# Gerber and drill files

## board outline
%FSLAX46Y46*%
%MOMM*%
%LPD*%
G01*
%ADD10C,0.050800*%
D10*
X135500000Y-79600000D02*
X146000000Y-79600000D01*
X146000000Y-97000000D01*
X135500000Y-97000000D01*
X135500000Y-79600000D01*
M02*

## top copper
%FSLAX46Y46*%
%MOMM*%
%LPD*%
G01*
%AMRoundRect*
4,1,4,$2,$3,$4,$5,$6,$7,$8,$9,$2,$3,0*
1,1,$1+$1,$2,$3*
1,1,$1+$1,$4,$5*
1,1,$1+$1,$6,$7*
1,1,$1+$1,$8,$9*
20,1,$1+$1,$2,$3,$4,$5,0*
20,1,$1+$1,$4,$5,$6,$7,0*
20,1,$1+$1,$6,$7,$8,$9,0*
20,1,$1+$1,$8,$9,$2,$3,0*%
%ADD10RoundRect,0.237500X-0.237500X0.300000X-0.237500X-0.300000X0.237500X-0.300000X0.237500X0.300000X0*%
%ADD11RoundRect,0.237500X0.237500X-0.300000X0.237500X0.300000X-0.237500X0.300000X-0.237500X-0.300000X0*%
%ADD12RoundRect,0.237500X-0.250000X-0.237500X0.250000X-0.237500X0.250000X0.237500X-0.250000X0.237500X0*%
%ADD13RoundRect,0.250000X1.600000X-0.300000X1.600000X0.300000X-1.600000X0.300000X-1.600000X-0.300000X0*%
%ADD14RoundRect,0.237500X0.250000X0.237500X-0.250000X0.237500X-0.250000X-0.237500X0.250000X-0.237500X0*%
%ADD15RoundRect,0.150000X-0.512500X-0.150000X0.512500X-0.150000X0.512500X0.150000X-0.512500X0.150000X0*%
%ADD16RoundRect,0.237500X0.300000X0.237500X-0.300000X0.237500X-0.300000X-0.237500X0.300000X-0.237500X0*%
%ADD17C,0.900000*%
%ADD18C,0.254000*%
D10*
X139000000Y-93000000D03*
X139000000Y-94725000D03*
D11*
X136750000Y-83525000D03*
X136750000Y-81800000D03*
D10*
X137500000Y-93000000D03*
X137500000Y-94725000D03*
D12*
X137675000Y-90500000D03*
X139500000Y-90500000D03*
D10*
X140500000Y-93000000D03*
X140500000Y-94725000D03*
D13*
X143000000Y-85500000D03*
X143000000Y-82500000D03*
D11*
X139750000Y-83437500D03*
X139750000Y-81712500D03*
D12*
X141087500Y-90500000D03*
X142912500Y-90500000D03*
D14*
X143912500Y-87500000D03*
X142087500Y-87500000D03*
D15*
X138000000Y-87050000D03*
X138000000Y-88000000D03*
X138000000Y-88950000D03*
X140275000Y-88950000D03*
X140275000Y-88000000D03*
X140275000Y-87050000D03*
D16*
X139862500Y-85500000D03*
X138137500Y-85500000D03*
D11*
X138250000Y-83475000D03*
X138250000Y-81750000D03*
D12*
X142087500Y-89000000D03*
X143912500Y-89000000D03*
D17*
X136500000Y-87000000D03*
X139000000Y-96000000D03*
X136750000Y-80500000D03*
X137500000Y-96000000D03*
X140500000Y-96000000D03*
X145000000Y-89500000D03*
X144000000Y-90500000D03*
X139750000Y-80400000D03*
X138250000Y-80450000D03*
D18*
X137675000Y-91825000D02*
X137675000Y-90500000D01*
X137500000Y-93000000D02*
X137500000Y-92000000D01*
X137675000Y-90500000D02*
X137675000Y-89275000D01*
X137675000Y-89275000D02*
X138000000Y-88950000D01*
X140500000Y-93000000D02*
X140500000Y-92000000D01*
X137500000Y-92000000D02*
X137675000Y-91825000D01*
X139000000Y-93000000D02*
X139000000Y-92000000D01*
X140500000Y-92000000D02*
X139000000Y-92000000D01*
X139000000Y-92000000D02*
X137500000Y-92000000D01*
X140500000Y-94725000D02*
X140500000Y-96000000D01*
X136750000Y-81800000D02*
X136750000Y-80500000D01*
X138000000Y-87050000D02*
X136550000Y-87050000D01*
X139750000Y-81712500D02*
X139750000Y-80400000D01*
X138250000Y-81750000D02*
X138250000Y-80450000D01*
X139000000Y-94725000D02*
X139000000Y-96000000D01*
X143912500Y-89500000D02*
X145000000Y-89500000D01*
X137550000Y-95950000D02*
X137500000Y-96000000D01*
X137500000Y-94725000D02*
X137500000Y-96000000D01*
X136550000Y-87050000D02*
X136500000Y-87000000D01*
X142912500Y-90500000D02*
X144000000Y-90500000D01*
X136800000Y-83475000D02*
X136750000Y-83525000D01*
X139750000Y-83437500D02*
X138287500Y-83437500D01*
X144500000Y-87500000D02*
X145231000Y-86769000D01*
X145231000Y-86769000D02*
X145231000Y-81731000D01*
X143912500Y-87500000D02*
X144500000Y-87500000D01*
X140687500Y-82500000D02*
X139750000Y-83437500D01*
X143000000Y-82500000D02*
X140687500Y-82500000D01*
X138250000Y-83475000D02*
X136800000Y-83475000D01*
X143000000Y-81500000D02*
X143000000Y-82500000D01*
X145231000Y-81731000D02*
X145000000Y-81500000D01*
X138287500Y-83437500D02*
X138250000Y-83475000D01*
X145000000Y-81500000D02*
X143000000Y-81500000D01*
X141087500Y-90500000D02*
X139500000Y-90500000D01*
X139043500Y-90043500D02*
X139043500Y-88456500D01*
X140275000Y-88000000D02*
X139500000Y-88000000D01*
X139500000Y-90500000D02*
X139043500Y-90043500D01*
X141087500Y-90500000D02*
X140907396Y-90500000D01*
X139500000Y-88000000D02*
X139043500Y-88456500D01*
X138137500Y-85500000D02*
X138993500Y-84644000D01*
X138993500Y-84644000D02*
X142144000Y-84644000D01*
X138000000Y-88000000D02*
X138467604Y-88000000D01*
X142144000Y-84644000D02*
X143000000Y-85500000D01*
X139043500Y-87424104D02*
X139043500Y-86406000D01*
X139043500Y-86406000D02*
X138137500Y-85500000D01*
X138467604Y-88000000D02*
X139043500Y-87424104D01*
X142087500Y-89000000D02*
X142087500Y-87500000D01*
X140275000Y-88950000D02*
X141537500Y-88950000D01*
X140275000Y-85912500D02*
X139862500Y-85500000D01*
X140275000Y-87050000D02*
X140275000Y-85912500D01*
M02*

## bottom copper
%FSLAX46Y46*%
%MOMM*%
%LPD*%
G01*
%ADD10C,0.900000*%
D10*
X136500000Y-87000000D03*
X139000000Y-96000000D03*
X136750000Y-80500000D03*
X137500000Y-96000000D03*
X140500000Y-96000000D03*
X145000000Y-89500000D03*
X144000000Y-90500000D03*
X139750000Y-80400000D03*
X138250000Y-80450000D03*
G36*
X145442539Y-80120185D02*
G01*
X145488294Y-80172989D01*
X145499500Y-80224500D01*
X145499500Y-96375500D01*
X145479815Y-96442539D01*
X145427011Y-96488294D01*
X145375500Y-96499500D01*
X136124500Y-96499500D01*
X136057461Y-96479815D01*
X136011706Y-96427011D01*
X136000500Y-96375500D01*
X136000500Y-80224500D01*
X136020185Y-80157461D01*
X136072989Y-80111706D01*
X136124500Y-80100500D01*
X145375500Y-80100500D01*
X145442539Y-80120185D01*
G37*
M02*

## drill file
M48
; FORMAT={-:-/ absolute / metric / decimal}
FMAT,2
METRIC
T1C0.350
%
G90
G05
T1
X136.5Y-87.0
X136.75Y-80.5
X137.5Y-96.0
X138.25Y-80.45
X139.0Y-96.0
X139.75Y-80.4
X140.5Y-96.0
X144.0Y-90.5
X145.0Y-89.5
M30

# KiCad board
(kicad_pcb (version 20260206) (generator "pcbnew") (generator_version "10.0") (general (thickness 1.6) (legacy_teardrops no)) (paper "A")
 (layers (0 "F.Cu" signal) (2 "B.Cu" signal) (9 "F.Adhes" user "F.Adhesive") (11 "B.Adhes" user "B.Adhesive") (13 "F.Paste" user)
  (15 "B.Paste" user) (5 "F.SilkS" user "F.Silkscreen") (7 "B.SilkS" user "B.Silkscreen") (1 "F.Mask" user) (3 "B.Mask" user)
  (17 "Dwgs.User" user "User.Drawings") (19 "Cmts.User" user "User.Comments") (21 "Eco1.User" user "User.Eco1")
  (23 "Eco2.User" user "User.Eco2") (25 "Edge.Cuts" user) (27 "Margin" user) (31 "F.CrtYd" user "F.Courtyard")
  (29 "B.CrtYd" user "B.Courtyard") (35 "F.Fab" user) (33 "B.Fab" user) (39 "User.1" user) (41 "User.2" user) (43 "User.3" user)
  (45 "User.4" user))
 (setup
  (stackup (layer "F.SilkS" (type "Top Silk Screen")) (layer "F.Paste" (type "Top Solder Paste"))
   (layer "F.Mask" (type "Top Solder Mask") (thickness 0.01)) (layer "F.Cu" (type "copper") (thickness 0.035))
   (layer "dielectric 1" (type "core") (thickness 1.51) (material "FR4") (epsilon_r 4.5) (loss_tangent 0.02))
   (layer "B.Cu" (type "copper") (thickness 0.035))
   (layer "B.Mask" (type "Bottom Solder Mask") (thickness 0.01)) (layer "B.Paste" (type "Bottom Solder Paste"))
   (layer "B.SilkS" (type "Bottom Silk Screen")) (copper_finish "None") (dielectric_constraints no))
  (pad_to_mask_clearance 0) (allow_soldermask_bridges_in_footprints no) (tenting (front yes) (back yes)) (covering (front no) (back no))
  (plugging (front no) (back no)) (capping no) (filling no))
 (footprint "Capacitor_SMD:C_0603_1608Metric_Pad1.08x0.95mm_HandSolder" (layer "F.Cu") (at 139 93.8625 -90)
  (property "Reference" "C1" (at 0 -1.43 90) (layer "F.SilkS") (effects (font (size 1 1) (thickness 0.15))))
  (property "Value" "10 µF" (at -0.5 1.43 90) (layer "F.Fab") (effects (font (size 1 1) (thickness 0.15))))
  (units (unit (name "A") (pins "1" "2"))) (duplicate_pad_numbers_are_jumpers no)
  (pad "1" smd roundrect (at -0.8625 0 270) (size 1.075 0.95) (layers "F.Cu" "F.Mask" "F.Paste") (roundrect_rratio 0.25) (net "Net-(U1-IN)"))
  (pad "2" smd roundrect (at 0.8625 0 270) (size 1.075 0.95) (layers "F.Cu" "F.Mask" "F.Paste") (roundrect_rratio 0.25) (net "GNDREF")))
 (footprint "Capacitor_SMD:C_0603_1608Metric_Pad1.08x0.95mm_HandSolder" (layer "F.Cu") (at 136.75 82.6625 90)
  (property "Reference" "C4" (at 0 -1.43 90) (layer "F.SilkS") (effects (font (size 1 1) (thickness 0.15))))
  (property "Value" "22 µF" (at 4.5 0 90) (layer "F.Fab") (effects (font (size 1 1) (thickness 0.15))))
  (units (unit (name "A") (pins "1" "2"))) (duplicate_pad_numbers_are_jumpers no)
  (pad "1" smd roundrect (at -0.8625 0 90) (size 1.075 0.95) (layers "F.Cu" "F.Mask" "F.Paste") (roundrect_rratio 0.25)
   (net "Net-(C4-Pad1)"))
  (pad "2" smd roundrect (at 0.8625 0 90) (size 1.075 0.95) (layers "F.Cu" "F.Mask" "F.Paste") (roundrect_rratio 0.25) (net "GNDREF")))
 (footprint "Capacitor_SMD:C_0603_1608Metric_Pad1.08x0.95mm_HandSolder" (layer "F.Cu") (at 137.5 93.8625 -90)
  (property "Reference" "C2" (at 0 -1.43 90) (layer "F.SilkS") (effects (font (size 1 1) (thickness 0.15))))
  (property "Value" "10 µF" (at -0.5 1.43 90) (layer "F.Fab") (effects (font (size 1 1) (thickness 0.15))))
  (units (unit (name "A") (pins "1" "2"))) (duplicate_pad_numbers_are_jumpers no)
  (pad "1" smd roundrect (at -0.8625 0 270) (size 1.075 0.95) (layers "F.Cu" "F.Mask" "F.Paste") (roundrect_rratio 0.25) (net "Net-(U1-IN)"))
  (pad "2" smd roundrect (at 0.8625 0 270) (size 1.075 0.95) (layers "F.Cu" "F.Mask" "F.Paste") (roundrect_rratio 0.25) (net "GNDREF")))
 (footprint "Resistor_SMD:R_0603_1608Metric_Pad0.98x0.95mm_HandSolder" (layer "F.Cu") (at 138.5875 90.5)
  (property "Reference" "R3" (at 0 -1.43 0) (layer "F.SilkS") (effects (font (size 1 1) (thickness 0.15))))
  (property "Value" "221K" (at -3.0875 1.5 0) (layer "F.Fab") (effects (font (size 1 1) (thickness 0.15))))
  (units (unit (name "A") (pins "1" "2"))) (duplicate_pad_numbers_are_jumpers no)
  (pad "1" smd roundrect (at -0.9125 0) (size 0.975 0.95) (layers "F.Cu" "F.Mask" "F.Paste") (roundrect_rratio 0.25) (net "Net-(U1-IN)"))
  (pad "2" smd roundrect (at 0.9125 0) (size 0.975 0.95) (layers "F.Cu" "F.Mask" "F.Paste") (roundrect_rratio 0.25) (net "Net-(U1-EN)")))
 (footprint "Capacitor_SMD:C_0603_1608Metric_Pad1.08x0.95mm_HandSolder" (layer "F.Cu") (at 140.5 93.8625 -90)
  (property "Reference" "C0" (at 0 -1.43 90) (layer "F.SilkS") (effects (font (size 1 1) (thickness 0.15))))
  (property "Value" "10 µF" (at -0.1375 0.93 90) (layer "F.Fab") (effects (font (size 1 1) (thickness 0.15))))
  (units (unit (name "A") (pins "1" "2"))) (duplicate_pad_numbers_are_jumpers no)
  (pad "1" smd roundrect (at -0.8625 0 270) (size 1.075 0.95) (layers "F.Cu" "F.Mask" "F.Paste") (roundrect_rratio 0.25) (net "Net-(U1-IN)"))
  (pad "2" smd roundrect (at 0.8625 0 270) (size 1.075 0.95) (layers "F.Cu" "F.Mask" "F.Paste") (roundrect_rratio 0.25) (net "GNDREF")))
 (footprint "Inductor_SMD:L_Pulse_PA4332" (layer "F.Cu") (at 143 84 90)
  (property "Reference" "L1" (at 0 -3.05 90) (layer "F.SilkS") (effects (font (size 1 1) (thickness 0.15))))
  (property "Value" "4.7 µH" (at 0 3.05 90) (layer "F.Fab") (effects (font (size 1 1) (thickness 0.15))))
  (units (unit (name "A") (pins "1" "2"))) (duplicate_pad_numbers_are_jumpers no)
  (pad "1" smd roundrect (at -1.5 0 90) (size 1.1 3.7) (layers "F.Cu" "F.Mask" "F.Paste") (roundrect_rratio 0.227273) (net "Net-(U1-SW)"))
  (pad "2" smd roundrect (at 1.5 0 90) (size 1.1 3.7) (layers "F.Cu" "F.Mask" "F.Paste") (roundrect_rratio 0.227273) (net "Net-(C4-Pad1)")))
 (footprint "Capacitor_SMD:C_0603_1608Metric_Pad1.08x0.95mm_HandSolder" (layer "F.Cu") (at 139.75 82.575 90)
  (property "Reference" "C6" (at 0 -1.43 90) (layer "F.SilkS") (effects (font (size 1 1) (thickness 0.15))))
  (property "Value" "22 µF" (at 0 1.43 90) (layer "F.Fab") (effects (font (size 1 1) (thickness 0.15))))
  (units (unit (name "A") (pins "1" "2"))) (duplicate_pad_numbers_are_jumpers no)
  (pad "1" smd roundrect (at -0.8625 0 90) (size 1.075 0.95) (layers "F.Cu" "F.Mask" "F.Paste") (roundrect_rratio 0.25)
   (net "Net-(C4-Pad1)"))
  (pad "2" smd roundrect (at 0.8625 0 90) (size 1.075 0.95) (layers "F.Cu" "F.Mask" "F.Paste") (roundrect_rratio 0.25) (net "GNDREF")))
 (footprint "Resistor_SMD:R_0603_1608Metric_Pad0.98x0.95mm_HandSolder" (layer "F.Cu") (at 142 90.5)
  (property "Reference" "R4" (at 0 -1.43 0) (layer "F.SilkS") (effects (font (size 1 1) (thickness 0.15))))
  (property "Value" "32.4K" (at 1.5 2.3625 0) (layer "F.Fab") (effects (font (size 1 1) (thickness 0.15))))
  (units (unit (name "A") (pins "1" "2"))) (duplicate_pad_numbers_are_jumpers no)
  (pad "1" smd roundrect (at -0.9125 0) (size 0.975 0.95) (layers "F.Cu" "F.Mask" "F.Paste") (roundrect_rratio 0.25) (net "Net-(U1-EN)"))
  (pad "2" smd roundrect (at 0.9125 0) (size 0.975 0.95) (layers "F.Cu" "F.Mask" "F.Paste") (roundrect_rratio 0.25) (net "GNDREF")))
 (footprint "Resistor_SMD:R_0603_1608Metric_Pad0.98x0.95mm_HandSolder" (layer "F.Cu") (at 143 87.5 180)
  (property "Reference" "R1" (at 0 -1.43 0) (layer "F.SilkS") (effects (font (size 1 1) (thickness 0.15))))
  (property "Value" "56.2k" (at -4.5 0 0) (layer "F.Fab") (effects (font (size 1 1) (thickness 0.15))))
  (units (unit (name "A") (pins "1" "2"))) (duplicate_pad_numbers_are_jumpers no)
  (pad "1" smd roundrect (at -0.9125 0 180) (size 0.975 0.95) (layers "F.Cu" "F.Mask" "F.Paste") (roundrect_rratio 0.25)
   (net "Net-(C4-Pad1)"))
  (pad "2" smd roundrect (at 0.9125 0 180) (size 0.975 0.95) (layers "F.Cu" "F.Mask" "F.Paste") (roundrect_rratio 0.25) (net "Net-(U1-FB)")))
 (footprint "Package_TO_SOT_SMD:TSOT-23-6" (layer "F.Cu") (at 139.1375 88)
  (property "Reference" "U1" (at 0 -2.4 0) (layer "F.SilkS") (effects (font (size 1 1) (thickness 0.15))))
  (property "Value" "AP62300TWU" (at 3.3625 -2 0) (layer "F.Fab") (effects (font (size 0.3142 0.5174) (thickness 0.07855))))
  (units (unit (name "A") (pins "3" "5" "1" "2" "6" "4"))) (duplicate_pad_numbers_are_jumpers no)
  (pad "1" smd roundrect (at -1.1375 -0.95) (size 1.325 0.6) (layers "F.Cu" "F.Mask" "F.Paste") (roundrect_rratio 0.25) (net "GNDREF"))
  (pad "2" smd roundrect (at -1.1375 0) (size 1.325 0.6) (layers "F.Cu" "F.Mask" "F.Paste") (roundrect_rratio 0.25) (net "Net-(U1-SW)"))
  (pad "3" smd roundrect (at -1.1375 0.95) (size 1.325 0.6) (layers "F.Cu" "F.Mask" "F.Paste") (roundrect_rratio 0.25) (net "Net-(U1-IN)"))
  (pad "4" smd roundrect (at 1.1375 0.95) (size 1.325 0.6) (layers "F.Cu" "F.Mask" "F.Paste") (roundrect_rratio 0.25) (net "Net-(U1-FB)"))
  (pad "5" smd roundrect (at 1.1375 0) (size 1.325 0.6) (layers "F.Cu" "F.Mask" "F.Paste") (roundrect_rratio 0.25) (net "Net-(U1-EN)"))
  (pad "6" smd roundrect (at 1.1375 -0.95) (size 1.325 0.6) (layers "F.Cu" "F.Mask" "F.Paste") (roundrect_rratio 0.25) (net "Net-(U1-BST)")))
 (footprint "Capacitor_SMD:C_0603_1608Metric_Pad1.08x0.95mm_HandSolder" (layer "F.Cu") (at 139 85.5 180)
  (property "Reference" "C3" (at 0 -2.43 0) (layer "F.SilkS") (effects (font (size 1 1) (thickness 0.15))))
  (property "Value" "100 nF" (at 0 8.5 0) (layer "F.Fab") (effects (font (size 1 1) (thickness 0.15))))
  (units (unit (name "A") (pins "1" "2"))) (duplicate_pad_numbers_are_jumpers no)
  (pad "1" smd roundrect (at -0.8625 0 180) (size 1.075 0.95) (layers "F.Cu" "F.Mask" "F.Paste") (roundrect_rratio 0.25)
   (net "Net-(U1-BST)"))
  (pad "2" smd roundrect (at 0.8625 0 180) (size 1.075 0.95) (layers "F.Cu" "F.Mask" "F.Paste") (roundrect_rratio 0.25) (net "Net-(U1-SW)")))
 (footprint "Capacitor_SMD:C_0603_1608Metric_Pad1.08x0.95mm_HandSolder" (layer "F.Cu") (at 138.25 82.6125 90)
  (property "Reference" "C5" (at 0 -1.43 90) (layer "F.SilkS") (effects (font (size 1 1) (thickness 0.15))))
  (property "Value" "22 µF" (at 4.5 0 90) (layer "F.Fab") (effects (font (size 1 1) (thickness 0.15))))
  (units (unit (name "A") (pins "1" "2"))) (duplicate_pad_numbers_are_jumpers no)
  (pad "1" smd roundrect (at -0.8625 0 90) (size 1.075 0.95) (layers "F.Cu" "F.Mask" "F.Paste") (roundrect_rratio 0.25)
   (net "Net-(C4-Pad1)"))
  (pad "2" smd roundrect (at 0.8625 0 90) (size 1.075 0.95) (layers "F.Cu" "F.Mask" "F.Paste") (roundrect_rratio 0.25) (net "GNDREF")))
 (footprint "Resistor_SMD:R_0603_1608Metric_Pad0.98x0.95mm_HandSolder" (layer "F.Cu") (at 143 89)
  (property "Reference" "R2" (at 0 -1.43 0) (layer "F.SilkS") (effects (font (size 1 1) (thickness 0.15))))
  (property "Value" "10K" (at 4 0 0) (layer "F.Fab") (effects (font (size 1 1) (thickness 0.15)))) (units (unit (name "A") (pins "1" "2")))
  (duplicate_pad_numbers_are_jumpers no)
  (pad "1" smd roundrect (at -0.9125 0) (size 0.975 0.95) (layers "F.Cu" "F.Mask" "F.Paste") (roundrect_rratio 0.25) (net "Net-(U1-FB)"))
  (pad "2" smd roundrect (at 0.9125 0) (size 0.975 0.95) (layers "F.Cu" "F.Mask" "F.Paste") (roundrect_rratio 0.25) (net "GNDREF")))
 (gr_rect (start 135.5 79.6) (end 146 97) (stroke (width 0.0508) (type solid)) (fill no) (layer "Edge.Cuts"))
 (segment (start 137.675 91.825) (end 137.675 90.5) (width 0.254) (layer "F.Cu") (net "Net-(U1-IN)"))
 (segment (start 137.5 93) (end 137.5 92) (width 0.254) (layer "F.Cu") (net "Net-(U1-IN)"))
 (segment (start 137.675 90.5) (end 137.675 89.275) (width 0.254) (layer "F.Cu") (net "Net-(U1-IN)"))
 (segment (start 137.675 89.275) (end 138 88.95) (width 0.254) (layer "F.Cu") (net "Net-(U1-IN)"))
 (segment (start 140.5 93) (end 140.5 92) (width 0.254) (layer "F.Cu") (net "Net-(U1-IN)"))
 (segment (start 137.5 92) (end 137.675 91.825) (width 0.254) (layer "F.Cu") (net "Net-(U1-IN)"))
 (segment (start 139 93) (end 139 92) (width 0.254) (layer "F.Cu") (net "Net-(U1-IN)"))
 (segment (start 140.5 92) (end 139 92) (width 0.254) (layer "F.Cu") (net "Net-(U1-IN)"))
 (segment (start 139 92) (end 137.5 92) (width 0.254) (layer "F.Cu") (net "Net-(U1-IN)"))
 (segment (start 140.5 94.725) (end 140.5 96) (width 0.254) (layer "F.Cu") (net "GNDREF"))
 (segment (start 136.75 81.8) (end 136.75 80.5) (width 0.254) (layer "F.Cu") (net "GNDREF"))
 (segment (start 138 87.05) (end 136.55 87.05) (width 0.254) (layer "F.Cu") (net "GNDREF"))
 (segment (start 139.75 81.7125) (end 139.75 80.4) (width 0.254) (layer "F.Cu") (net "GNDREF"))
 (segment (start 138.25 81.75) (end 138.25 80.45) (width 0.254) (layer "F.Cu") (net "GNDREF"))
 (segment (start 139 94.725) (end 139 96) (width 0.254) (layer "F.Cu") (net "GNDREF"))
 (segment (start 143.9125 89.5) (end 145 89.5) (width 0.254) (layer "F.Cu") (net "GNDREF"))
 (segment (start 137.55 95.95) (end 137.5 96) (width 0.254) (layer "F.Cu") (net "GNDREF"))
 (segment (start 137.5 94.725) (end 137.5 96) (width 0.254) (layer "F.Cu") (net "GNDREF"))
 (segment (start 136.55 87.05) (end 136.5 87) (width 0.254) (layer "F.Cu") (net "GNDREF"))
 (segment (start 142.9125 90.5) (end 144 90.5) (width 0.254) (layer "F.Cu") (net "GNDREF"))
 (via (at 136.5 87) (size 0.9) (drill 0.35) (layers "F.Cu" "B.Cu") (free yes) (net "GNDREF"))
 (via (at 139 96) (size 0.9) (drill 0.35) (layers "F.Cu" "B.Cu") (free yes) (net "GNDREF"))
 (via (at 136.75 80.5) (size 0.9) (drill 0.35) (layers "F.Cu" "B.Cu") (free yes) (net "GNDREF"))
 (via (at 137.5 96) (size 0.9) (drill 0.35) (layers "F.Cu" "B.Cu") (free yes) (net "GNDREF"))
 (via (at 140.5 96) (size 0.9) (drill 0.35) (layers "F.Cu" "B.Cu") (free yes) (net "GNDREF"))
 (via (at 145 89.5) (size 0.9) (drill 0.35) (layers "F.Cu" "B.Cu") (free yes) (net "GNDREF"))
 (via (at 144 90.5) (size 0.9) (drill 0.35) (layers "F.Cu" "B.Cu") (free yes) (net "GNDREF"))
 (via (at 139.75 80.4) (size 0.9) (drill 0.35) (layers "F.Cu" "B.Cu") (free yes) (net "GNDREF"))
 (via (at 138.25 80.45) (size 0.9) (drill 0.35) (layers "F.Cu" "B.Cu") (free yes) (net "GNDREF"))
 (segment (start 136.8 83.475) (end 136.75 83.525) (width 0.254) (layer "F.Cu") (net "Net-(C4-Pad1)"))
 (segment (start 139.75 83.4375) (end 138.2875 83.4375) (width 0.254) (layer "F.Cu") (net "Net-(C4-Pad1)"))
 (segment (start 144.5 87.5) (end 145.231 86.769) (width 0.254) (layer "F.Cu") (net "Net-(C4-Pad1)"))
 (segment (start 145.231 86.769) (end 145.231 81.731) (width 0.254) (layer "F.Cu") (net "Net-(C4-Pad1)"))
 (segment (start 143.9125 87.5) (end 144.5 87.5) (width 0.254) (layer "F.Cu") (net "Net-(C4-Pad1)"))
 (segment (start 140.6875 82.5) (end 139.75 83.4375) (width 0.254) (layer "F.Cu") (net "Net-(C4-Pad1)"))
 (segment (start 143 82.5) (end 140.6875 82.5) (width 0.254) (layer "F.Cu") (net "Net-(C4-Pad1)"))
 (segment (start 138.25 83.475) (end 136.8 83.475) (width 0.254) (layer "F.Cu") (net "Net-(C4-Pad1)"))
 (segment (start 143 81.5) (end 143 82.5) (width 0.254) (layer "F.Cu") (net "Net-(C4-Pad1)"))
 (segment (start 145.231 81.731) (end 145 81.5) (width 0.254) (layer "F.Cu") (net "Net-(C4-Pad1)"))
 (segment (start 138.2875 83.4375) (end 138.25 83.475) (width 0.254) (layer "F.Cu") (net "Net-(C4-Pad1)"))
 (segment (start 145 81.5) (end 143 81.5) (width 0.254) (layer "F.Cu") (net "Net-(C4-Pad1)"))
 (segment (start 141.0875 90.5) (end 139.5 90.5) (width 0.254) (layer "F.Cu") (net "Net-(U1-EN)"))
 (segment (start 139.0435 90.0435) (end 139.0435 88.4565) (width 0.254) (layer "F.Cu") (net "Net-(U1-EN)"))
 (segment (start 140.275 88) (end 139.5 88) (width 0.254) (layer "F.Cu") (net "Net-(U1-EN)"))
 (segment (start 139.5 90.5) (end 139.0435 90.0435) (width 0.254) (layer "F.Cu") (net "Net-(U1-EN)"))
 (segment (start 141.0875 90.5) (end 140.907396 90.5) (width 0.254) (layer "F.Cu") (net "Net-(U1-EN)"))
 (segment (start 139.5 88) (end 139.0435 88.4565) (width 0.254) (layer "F.Cu") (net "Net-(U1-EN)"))
 (segment (start 138.1375 85.5) (end 138.9935 84.644) (width 0.254) (layer "F.Cu") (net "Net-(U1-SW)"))
 (segment (start 138.9935 84.644) (end 142.144 84.644) (width 0.254) (layer "F.Cu") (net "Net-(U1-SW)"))
 (segment (start 138 88) (end 138.467604 88) (width 0.254) (layer "F.Cu") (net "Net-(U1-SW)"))
 (segment (start 142.144 84.644) (end 143 85.5) (width 0.254) (layer "F.Cu") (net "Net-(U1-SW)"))
 (segment (start 139.0435 87.424104) (end 139.0435 86.406) (width 0.254) (layer "F.Cu") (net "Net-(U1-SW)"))
 (segment (start 139.0435 86.406) (end 138.1375 85.5) (width 0.254) (layer "F.Cu") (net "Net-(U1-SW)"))
 (segment (start 138.467604 88) (end 139.0435 87.424104) (width 0.254) (layer "F.Cu") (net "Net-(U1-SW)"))
 (segment (start 142.0875 89) (end 142.0875 87.5) (width 0.254) (layer "F.Cu") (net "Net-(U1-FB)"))
 (segment (start 140.275 88.95) (end 141.5375 88.95) (width 0.254) (layer "F.Cu") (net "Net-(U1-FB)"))
 (segment (start 140.275 85.9125) (end 139.8625 85.5) (width 0.254) (layer "F.Cu") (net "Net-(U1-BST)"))
 (segment (start 140.275 87.05) (end 140.275 85.9125) (width 0.254) (layer "F.Cu") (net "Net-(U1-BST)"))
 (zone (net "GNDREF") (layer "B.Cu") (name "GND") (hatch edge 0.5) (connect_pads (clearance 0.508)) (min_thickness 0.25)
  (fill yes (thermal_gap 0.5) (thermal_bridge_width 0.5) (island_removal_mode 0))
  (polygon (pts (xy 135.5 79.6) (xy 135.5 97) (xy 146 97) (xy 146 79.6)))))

